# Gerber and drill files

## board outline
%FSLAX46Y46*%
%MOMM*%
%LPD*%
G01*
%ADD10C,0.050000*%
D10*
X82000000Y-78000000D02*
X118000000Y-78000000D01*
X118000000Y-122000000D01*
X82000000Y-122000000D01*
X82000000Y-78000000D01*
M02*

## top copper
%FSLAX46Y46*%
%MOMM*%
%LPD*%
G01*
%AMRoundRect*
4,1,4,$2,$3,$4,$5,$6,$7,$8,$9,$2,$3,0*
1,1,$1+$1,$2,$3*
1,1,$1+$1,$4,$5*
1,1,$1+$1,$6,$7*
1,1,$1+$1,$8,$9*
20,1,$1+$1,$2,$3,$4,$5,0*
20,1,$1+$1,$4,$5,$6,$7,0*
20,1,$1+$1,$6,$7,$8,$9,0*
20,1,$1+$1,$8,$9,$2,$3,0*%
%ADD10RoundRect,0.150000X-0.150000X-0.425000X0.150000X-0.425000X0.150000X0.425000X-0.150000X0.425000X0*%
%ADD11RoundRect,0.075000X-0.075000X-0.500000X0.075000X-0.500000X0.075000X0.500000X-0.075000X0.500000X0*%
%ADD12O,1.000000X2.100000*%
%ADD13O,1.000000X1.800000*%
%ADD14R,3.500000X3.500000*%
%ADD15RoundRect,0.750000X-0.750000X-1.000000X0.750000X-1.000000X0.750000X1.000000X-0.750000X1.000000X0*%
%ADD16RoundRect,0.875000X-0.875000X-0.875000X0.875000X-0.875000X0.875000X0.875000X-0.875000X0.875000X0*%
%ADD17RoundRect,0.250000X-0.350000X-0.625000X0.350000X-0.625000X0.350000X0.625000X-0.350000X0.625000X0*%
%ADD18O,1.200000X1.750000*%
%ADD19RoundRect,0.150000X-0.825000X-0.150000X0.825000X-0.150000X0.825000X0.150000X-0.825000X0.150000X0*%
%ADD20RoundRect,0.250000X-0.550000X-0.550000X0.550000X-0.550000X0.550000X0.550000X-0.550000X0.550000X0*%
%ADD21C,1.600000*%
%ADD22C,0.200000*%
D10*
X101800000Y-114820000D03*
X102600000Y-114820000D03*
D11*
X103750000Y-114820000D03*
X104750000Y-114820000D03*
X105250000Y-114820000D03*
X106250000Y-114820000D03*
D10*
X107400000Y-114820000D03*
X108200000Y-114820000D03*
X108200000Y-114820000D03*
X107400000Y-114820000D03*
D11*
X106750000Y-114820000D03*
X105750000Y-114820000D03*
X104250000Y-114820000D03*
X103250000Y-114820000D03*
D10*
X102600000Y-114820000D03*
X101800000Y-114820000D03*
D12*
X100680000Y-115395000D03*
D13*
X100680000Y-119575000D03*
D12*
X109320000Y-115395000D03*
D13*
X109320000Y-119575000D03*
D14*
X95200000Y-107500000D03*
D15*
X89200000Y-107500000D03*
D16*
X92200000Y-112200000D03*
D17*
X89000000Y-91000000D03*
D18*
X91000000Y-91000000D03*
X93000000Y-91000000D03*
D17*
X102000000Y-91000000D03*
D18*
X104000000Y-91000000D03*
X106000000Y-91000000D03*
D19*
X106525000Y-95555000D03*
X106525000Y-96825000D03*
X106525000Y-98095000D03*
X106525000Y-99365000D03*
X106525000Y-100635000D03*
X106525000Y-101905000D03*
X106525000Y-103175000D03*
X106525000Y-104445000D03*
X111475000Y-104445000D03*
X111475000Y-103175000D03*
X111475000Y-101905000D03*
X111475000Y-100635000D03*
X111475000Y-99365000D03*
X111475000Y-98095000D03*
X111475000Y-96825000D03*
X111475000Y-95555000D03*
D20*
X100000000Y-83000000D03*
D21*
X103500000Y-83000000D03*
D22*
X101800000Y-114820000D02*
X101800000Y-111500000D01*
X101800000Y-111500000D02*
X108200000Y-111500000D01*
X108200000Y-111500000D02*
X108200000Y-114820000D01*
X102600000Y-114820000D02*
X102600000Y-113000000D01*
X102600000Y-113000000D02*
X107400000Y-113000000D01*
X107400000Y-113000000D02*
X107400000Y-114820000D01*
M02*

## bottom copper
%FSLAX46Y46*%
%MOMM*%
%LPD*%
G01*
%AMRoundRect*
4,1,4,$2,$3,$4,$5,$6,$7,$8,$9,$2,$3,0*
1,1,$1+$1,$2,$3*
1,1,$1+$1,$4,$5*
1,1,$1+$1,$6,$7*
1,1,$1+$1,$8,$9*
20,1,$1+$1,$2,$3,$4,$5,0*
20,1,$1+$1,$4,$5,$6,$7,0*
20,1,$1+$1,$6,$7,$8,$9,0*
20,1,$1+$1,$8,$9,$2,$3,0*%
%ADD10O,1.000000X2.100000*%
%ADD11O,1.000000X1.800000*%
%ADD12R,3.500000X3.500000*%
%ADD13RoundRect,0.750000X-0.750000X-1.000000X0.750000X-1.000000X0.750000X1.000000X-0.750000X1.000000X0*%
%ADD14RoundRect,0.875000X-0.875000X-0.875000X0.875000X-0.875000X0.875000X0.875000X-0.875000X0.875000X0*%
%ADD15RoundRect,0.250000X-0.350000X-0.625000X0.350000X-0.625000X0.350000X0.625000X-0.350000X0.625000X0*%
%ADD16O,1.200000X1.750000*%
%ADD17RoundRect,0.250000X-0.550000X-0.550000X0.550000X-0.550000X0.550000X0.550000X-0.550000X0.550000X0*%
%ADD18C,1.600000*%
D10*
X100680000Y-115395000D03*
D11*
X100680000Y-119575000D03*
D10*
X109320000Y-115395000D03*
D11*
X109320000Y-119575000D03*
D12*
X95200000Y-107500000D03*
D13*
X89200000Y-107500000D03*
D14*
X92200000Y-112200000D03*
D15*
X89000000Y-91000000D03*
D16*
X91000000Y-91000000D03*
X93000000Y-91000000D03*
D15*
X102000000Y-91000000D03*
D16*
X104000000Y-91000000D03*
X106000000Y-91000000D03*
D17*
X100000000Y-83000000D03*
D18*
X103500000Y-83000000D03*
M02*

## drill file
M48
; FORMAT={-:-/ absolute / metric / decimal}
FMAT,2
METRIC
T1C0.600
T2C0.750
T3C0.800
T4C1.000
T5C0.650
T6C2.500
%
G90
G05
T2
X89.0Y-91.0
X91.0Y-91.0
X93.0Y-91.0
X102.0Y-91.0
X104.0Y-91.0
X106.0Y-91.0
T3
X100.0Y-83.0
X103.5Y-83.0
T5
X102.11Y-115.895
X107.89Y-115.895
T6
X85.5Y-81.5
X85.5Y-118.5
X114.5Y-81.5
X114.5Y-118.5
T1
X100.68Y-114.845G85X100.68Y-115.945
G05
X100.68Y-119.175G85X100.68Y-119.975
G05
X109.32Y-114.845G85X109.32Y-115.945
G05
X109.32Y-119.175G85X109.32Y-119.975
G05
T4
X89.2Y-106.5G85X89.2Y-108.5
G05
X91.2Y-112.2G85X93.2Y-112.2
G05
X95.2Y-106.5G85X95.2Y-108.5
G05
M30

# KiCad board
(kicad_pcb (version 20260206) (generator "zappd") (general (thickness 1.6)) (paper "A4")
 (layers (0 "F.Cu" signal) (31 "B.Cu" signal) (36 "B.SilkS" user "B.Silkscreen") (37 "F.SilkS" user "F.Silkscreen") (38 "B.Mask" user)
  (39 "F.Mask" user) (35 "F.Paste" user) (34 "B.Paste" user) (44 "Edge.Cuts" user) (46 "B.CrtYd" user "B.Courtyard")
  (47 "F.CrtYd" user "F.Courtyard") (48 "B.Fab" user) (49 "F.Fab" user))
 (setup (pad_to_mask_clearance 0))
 (gr_rect (start 82.0 78.0) (end 118.0 122.0) (stroke (width 0.05) (type default)) (fill none) (layer "Edge.Cuts"))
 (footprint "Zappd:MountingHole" (layer "F.Cu") (at 85.5 81.5)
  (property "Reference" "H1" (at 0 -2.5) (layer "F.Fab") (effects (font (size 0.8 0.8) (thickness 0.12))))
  (pad "" np_thru_hole circle (at 0 0) (size 2.5 2.5) (drill 2.5) (layers "*.Cu" "*.Mask")))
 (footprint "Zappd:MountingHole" (layer "F.Cu") (at 114.5 81.5)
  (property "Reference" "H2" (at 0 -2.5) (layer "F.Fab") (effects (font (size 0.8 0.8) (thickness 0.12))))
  (pad "" np_thru_hole circle (at 0 0) (size 2.5 2.5) (drill 2.5) (layers "*.Cu" "*.Mask")))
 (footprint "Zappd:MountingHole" (layer "F.Cu") (at 114.5 118.5)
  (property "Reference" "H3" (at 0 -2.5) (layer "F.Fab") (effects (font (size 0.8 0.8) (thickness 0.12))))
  (pad "" np_thru_hole circle (at 0 0) (size 2.5 2.5) (drill 2.5) (layers "*.Cu" "*.Mask")))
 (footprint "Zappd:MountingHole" (layer "F.Cu") (at 85.5 118.5)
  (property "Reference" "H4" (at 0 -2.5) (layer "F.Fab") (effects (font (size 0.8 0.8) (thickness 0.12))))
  (pad "" np_thru_hole circle (at 0 0) (size 2.5 2.5) (drill 2.5) (layers "*.Cu" "*.Mask")))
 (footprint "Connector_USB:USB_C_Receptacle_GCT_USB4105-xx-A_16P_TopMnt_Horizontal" (layer "F.Cu") (at 105 118.5)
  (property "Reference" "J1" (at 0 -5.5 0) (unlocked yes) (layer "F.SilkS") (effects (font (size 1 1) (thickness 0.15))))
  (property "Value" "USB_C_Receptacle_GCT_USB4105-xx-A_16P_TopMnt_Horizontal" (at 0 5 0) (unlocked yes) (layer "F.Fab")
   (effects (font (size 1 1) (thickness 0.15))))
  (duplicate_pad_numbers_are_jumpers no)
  (pad "" np_thru_hole circle (at -2.89 -2.605) (size 0.65 0.65) (drill 0.65) (layers "*.Cu" "*.Mask"))
  (pad "" np_thru_hole circle (at 2.89 -2.605) (size 0.65 0.65) (drill 0.65) (layers "*.Cu" "*.Mask"))
  (pad "A1" smd roundrect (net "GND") (at -3.2 -3.68) (size 0.6 1.15) (layers "F.Cu" "F.Mask" "F.Paste") (roundrect_rratio 0.25))
  (pad "A4" smd roundrect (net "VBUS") (at -2.4 -3.68) (size 0.6 1.15) (layers "F.Cu" "F.Mask" "F.Paste") (roundrect_rratio 0.25))
  (pad "A5" smd roundrect (at -1.25 -3.68) (size 0.3 1.15) (layers "F.Cu" "F.Mask" "F.Paste") (roundrect_rratio 0.25))
  (pad "A6" smd roundrect (at -0.25 -3.68) (size 0.3 1.15) (layers "F.Cu" "F.Mask" "F.Paste") (roundrect_rratio 0.25))
  (pad "A7" smd roundrect (at 0.25 -3.68) (size 0.3 1.15) (layers "F.Cu" "F.Mask" "F.Paste") (roundrect_rratio 0.25))
  (pad "A8" smd roundrect (at 1.25 -3.68) (size 0.3 1.15) (layers "F.Cu" "F.Mask" "F.Paste") (roundrect_rratio 0.25))
  (pad "A9" smd roundrect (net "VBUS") (at 2.4 -3.68) (size 0.6 1.15) (layers "F.Cu" "F.Mask" "F.Paste") (roundrect_rratio 0.25))
  (pad "A12" smd roundrect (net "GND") (at 3.2 -3.68) (size 0.6 1.15) (layers "F.Cu" "F.Mask" "F.Paste") (roundrect_rratio 0.25))
  (pad "B1" smd roundrect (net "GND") (at 3.2 -3.68) (size 0.6 1.15) (layers "F.Cu" "F.Mask" "F.Paste") (roundrect_rratio 0.25))
  (pad "B4" smd roundrect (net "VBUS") (at 2.4 -3.68) (size 0.6 1.15) (layers "F.Cu" "F.Mask" "F.Paste") (roundrect_rratio 0.25))
  (pad "B5" smd roundrect (at 1.75 -3.68) (size 0.3 1.15) (layers "F.Cu" "F.Mask" "F.Paste") (roundrect_rratio 0.25))
  (pad "B6" smd roundrect (at 0.75 -3.68) (size 0.3 1.15) (layers "F.Cu" "F.Mask" "F.Paste") (roundrect_rratio 0.25))
  (pad "B7" smd roundrect (at -0.75 -3.68) (size 0.3 1.15) (layers "F.Cu" "F.Mask" "F.Paste") (roundrect_rratio 0.25))
  (pad "B8" smd roundrect (at -1.75 -3.68) (size 0.3 1.15) (layers "F.Cu" "F.Mask" "F.Paste") (roundrect_rratio 0.25))
  (pad "B9" smd roundrect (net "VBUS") (at -2.4 -3.68) (size 0.6 1.15) (layers "F.Cu" "F.Mask" "F.Paste") (roundrect_rratio 0.25))
  (pad "B12" smd roundrect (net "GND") (at -3.2 -3.68) (size 0.6 1.15) (layers "F.Cu" "F.Mask" "F.Paste") (roundrect_rratio 0.25))
  (pad "SH" thru_hole oval (at -4.32 -3.105) (size 1 2.1) (drill oval 0.6 1.7) (layers "*.Cu" "*.Mask" "F.Paste") (remove_unused_layers no))
  (pad "SH" thru_hole oval (at -4.32 1.075) (size 1 1.8) (drill oval 0.6 1.4) (layers "*.Cu" "*.Mask" "F.Paste") (remove_unused_layers no))
  (pad "SH" thru_hole oval (at 4.32 -3.105) (size 1 2.1) (drill oval 0.6 1.7) (layers "*.Cu" "*.Mask" "F.Paste") (remove_unused_layers no))
  (pad "SH" thru_hole oval (at 4.32 1.075) (size 1 1.8) (drill oval 0.6 1.4) (layers "*.Cu" "*.Mask" "F.Paste") (remove_unused_layers no)))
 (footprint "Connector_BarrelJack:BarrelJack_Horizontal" (layer "F.Cu") (at 95.2 107.5)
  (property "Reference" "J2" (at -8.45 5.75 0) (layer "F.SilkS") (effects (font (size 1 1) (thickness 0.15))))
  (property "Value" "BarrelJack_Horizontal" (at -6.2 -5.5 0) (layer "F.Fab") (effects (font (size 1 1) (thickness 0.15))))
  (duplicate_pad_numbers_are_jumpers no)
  (pad "1" thru_hole rect (at 0 0) (size 3.5 3.5) (drill oval 1 3) (layers "*.Cu" "*.Mask") (remove_unused_layers no))
  (pad "2" thru_hole roundrect (at -6 0) (size 3 3.5) (drill oval 1 3) (layers "*.Cu" "*.Mask") (remove_unused_layers no)
   (roundrect_rratio 0.25))
  (pad "3" thru_hole roundrect (at -3 4.7) (size 3.5 3.5) (drill oval 3 1) (layers "*.Cu" "*.Mask") (remove_unused_layers no)
   (roundrect_rratio 0.25)))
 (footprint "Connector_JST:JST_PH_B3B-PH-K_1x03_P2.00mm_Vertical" (layer "F.Cu") (at 89 91)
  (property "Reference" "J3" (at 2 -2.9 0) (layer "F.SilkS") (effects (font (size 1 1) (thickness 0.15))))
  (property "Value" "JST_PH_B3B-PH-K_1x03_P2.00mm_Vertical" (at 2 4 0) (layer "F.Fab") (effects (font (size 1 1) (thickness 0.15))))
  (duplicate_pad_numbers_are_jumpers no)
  (pad "1" thru_hole roundrect (at 0 0) (size 1.2 1.75) (drill 0.75) (layers "*.Cu" "*.Mask") (remove_unused_layers no)
   (roundrect_rratio 0.208333))
  (pad "2" thru_hole oval (at 2 0) (size 1.2 1.75) (drill 0.75) (layers "*.Cu" "*.Mask") (remove_unused_layers no))
  (pad "3" thru_hole oval (at 4 0) (size 1.2 1.75) (drill 0.75) (layers "*.Cu" "*.Mask") (remove_unused_layers no)))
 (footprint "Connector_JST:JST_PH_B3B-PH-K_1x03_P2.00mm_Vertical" (layer "F.Cu") (at 102 91)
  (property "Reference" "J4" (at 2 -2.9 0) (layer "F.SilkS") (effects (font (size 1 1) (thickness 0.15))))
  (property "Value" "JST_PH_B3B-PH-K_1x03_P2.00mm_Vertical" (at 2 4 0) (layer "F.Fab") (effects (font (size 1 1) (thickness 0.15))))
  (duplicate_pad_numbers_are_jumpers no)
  (pad "1" thru_hole roundrect (at 0 0) (size 1.2 1.75) (drill 0.75) (layers "*.Cu" "*.Mask") (remove_unused_layers no)
   (roundrect_rratio 0.208333))
  (pad "2" thru_hole oval (at 2 0) (size 1.2 1.75) (drill 0.75) (layers "*.Cu" "*.Mask") (remove_unused_layers no))
  (pad "3" thru_hole oval (at 4 0) (size 1.2 1.75) (drill 0.75) (layers "*.Cu" "*.Mask") (remove_unused_layers no)))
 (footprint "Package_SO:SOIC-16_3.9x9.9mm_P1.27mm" (layer "F.Cu") (at 109 100)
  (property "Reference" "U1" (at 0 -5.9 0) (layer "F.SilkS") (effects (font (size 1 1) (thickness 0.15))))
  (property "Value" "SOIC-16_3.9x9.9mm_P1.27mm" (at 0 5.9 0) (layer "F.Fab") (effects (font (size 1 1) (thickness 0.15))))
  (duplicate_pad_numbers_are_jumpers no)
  (pad "1" smd roundrect (at -2.475 -4.445) (size 1.95 0.6) (layers "F.Cu" "F.Mask" "F.Paste") (roundrect_rratio 0.25))
  (pad "2" smd roundrect (at -2.475 -3.175) (size 1.95 0.6) (layers "F.Cu" "F.Mask" "F.Paste") (roundrect_rratio 0.25))
  (pad "3" smd roundrect (at -2.475 -1.905) (size 1.95 0.6) (layers "F.Cu" "F.Mask" "F.Paste") (roundrect_rratio 0.25))
  (pad "4" smd roundrect (at -2.475 -0.635) (size 1.95 0.6) (layers "F.Cu" "F.Mask" "F.Paste") (roundrect_rratio 0.25))
  (pad "5" smd roundrect (at -2.475 0.635) (size 1.95 0.6) (layers "F.Cu" "F.Mask" "F.Paste") (roundrect_rratio 0.25))
  (pad "6" smd roundrect (at -2.475 1.905) (size 1.95 0.6) (layers "F.Cu" "F.Mask" "F.Paste") (roundrect_rratio 0.25))
  (pad "7" smd roundrect (at -2.475 3.175) (size 1.95 0.6) (layers "F.Cu" "F.Mask" "F.Paste") (roundrect_rratio 0.25))
  (pad "8" smd roundrect (at -2.475 4.445) (size 1.95 0.6) (layers "F.Cu" "F.Mask" "F.Paste") (roundrect_rratio 0.25))
  (pad "9" smd roundrect (at 2.475 4.445) (size 1.95 0.6) (layers "F.Cu" "F.Mask" "F.Paste") (roundrect_rratio 0.25))
  (pad "10" smd roundrect (at 2.475 3.175) (size 1.95 0.6) (layers "F.Cu" "F.Mask" "F.Paste") (roundrect_rratio 0.25))
  (pad "11" smd roundrect (at 2.475 1.905) (size 1.95 0.6) (layers "F.Cu" "F.Mask" "F.Paste") (roundrect_rratio 0.25))
  (pad "12" smd roundrect (at 2.475 0.635) (size 1.95 0.6) (layers "F.Cu" "F.Mask" "F.Paste") (roundrect_rratio 0.25))
  (pad "13" smd roundrect (at 2.475 -0.635) (size 1.95 0.6) (layers "F.Cu" "F.Mask" "F.Paste") (roundrect_rratio 0.25))
  (pad "14" smd roundrect (at 2.475 -1.905) (size 1.95 0.6) (layers "F.Cu" "F.Mask" "F.Paste") (roundrect_rratio 0.25))
  (pad "15" smd roundrect (at 2.475 -3.175) (size 1.95 0.6) (layers "F.Cu" "F.Mask" "F.Paste") (roundrect_rratio 0.25))
  (pad "16" smd roundrect (at 2.475 -4.445) (size 1.95 0.6) (layers "F.Cu" "F.Mask" "F.Paste") (roundrect_rratio 0.25)))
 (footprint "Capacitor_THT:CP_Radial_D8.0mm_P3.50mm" (layer "F.Cu") (at 100 83)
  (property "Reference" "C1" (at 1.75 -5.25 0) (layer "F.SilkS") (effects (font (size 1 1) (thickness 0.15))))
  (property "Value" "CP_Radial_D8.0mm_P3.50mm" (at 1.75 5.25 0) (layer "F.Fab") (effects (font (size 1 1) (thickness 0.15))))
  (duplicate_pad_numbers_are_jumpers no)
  (pad "1" thru_hole roundrect (at 0 0) (size 1.6 1.6) (drill 0.8) (layers "*.Cu" "*.Mask") (remove_unused_layers no)
   (roundrect_rratio 0.15625))
  (pad "2" thru_hole circle (at 3.5 0) (size 1.6 1.6) (drill 0.8) (layers "*.Cu" "*.Mask") (remove_unused_layers no)))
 (segment (start 101.8000 114.8200) (end 101.8000 111.5000) (width 0.2) (layer "F.Cu") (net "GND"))
 (segment (start 101.8000 111.5000) (end 108.2000 111.5000) (width 0.2) (layer "F.Cu") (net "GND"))
 (segment (start 108.2000 111.5000) (end 108.2000 114.8200) (width 0.2) (layer "F.Cu") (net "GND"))
 (segment (start 102.6000 114.8200) (end 102.6000 113.0000) (width 0.2) (layer "F.Cu") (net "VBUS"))
 (segment (start 102.6000 113.0000) (end 107.4000 113.0000) (width 0.2) (layer "F.Cu") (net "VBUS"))
 (segment (start 107.4000 113.0000) (end 107.4000 114.8200) (width 0.2) (layer "F.Cu") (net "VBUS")))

